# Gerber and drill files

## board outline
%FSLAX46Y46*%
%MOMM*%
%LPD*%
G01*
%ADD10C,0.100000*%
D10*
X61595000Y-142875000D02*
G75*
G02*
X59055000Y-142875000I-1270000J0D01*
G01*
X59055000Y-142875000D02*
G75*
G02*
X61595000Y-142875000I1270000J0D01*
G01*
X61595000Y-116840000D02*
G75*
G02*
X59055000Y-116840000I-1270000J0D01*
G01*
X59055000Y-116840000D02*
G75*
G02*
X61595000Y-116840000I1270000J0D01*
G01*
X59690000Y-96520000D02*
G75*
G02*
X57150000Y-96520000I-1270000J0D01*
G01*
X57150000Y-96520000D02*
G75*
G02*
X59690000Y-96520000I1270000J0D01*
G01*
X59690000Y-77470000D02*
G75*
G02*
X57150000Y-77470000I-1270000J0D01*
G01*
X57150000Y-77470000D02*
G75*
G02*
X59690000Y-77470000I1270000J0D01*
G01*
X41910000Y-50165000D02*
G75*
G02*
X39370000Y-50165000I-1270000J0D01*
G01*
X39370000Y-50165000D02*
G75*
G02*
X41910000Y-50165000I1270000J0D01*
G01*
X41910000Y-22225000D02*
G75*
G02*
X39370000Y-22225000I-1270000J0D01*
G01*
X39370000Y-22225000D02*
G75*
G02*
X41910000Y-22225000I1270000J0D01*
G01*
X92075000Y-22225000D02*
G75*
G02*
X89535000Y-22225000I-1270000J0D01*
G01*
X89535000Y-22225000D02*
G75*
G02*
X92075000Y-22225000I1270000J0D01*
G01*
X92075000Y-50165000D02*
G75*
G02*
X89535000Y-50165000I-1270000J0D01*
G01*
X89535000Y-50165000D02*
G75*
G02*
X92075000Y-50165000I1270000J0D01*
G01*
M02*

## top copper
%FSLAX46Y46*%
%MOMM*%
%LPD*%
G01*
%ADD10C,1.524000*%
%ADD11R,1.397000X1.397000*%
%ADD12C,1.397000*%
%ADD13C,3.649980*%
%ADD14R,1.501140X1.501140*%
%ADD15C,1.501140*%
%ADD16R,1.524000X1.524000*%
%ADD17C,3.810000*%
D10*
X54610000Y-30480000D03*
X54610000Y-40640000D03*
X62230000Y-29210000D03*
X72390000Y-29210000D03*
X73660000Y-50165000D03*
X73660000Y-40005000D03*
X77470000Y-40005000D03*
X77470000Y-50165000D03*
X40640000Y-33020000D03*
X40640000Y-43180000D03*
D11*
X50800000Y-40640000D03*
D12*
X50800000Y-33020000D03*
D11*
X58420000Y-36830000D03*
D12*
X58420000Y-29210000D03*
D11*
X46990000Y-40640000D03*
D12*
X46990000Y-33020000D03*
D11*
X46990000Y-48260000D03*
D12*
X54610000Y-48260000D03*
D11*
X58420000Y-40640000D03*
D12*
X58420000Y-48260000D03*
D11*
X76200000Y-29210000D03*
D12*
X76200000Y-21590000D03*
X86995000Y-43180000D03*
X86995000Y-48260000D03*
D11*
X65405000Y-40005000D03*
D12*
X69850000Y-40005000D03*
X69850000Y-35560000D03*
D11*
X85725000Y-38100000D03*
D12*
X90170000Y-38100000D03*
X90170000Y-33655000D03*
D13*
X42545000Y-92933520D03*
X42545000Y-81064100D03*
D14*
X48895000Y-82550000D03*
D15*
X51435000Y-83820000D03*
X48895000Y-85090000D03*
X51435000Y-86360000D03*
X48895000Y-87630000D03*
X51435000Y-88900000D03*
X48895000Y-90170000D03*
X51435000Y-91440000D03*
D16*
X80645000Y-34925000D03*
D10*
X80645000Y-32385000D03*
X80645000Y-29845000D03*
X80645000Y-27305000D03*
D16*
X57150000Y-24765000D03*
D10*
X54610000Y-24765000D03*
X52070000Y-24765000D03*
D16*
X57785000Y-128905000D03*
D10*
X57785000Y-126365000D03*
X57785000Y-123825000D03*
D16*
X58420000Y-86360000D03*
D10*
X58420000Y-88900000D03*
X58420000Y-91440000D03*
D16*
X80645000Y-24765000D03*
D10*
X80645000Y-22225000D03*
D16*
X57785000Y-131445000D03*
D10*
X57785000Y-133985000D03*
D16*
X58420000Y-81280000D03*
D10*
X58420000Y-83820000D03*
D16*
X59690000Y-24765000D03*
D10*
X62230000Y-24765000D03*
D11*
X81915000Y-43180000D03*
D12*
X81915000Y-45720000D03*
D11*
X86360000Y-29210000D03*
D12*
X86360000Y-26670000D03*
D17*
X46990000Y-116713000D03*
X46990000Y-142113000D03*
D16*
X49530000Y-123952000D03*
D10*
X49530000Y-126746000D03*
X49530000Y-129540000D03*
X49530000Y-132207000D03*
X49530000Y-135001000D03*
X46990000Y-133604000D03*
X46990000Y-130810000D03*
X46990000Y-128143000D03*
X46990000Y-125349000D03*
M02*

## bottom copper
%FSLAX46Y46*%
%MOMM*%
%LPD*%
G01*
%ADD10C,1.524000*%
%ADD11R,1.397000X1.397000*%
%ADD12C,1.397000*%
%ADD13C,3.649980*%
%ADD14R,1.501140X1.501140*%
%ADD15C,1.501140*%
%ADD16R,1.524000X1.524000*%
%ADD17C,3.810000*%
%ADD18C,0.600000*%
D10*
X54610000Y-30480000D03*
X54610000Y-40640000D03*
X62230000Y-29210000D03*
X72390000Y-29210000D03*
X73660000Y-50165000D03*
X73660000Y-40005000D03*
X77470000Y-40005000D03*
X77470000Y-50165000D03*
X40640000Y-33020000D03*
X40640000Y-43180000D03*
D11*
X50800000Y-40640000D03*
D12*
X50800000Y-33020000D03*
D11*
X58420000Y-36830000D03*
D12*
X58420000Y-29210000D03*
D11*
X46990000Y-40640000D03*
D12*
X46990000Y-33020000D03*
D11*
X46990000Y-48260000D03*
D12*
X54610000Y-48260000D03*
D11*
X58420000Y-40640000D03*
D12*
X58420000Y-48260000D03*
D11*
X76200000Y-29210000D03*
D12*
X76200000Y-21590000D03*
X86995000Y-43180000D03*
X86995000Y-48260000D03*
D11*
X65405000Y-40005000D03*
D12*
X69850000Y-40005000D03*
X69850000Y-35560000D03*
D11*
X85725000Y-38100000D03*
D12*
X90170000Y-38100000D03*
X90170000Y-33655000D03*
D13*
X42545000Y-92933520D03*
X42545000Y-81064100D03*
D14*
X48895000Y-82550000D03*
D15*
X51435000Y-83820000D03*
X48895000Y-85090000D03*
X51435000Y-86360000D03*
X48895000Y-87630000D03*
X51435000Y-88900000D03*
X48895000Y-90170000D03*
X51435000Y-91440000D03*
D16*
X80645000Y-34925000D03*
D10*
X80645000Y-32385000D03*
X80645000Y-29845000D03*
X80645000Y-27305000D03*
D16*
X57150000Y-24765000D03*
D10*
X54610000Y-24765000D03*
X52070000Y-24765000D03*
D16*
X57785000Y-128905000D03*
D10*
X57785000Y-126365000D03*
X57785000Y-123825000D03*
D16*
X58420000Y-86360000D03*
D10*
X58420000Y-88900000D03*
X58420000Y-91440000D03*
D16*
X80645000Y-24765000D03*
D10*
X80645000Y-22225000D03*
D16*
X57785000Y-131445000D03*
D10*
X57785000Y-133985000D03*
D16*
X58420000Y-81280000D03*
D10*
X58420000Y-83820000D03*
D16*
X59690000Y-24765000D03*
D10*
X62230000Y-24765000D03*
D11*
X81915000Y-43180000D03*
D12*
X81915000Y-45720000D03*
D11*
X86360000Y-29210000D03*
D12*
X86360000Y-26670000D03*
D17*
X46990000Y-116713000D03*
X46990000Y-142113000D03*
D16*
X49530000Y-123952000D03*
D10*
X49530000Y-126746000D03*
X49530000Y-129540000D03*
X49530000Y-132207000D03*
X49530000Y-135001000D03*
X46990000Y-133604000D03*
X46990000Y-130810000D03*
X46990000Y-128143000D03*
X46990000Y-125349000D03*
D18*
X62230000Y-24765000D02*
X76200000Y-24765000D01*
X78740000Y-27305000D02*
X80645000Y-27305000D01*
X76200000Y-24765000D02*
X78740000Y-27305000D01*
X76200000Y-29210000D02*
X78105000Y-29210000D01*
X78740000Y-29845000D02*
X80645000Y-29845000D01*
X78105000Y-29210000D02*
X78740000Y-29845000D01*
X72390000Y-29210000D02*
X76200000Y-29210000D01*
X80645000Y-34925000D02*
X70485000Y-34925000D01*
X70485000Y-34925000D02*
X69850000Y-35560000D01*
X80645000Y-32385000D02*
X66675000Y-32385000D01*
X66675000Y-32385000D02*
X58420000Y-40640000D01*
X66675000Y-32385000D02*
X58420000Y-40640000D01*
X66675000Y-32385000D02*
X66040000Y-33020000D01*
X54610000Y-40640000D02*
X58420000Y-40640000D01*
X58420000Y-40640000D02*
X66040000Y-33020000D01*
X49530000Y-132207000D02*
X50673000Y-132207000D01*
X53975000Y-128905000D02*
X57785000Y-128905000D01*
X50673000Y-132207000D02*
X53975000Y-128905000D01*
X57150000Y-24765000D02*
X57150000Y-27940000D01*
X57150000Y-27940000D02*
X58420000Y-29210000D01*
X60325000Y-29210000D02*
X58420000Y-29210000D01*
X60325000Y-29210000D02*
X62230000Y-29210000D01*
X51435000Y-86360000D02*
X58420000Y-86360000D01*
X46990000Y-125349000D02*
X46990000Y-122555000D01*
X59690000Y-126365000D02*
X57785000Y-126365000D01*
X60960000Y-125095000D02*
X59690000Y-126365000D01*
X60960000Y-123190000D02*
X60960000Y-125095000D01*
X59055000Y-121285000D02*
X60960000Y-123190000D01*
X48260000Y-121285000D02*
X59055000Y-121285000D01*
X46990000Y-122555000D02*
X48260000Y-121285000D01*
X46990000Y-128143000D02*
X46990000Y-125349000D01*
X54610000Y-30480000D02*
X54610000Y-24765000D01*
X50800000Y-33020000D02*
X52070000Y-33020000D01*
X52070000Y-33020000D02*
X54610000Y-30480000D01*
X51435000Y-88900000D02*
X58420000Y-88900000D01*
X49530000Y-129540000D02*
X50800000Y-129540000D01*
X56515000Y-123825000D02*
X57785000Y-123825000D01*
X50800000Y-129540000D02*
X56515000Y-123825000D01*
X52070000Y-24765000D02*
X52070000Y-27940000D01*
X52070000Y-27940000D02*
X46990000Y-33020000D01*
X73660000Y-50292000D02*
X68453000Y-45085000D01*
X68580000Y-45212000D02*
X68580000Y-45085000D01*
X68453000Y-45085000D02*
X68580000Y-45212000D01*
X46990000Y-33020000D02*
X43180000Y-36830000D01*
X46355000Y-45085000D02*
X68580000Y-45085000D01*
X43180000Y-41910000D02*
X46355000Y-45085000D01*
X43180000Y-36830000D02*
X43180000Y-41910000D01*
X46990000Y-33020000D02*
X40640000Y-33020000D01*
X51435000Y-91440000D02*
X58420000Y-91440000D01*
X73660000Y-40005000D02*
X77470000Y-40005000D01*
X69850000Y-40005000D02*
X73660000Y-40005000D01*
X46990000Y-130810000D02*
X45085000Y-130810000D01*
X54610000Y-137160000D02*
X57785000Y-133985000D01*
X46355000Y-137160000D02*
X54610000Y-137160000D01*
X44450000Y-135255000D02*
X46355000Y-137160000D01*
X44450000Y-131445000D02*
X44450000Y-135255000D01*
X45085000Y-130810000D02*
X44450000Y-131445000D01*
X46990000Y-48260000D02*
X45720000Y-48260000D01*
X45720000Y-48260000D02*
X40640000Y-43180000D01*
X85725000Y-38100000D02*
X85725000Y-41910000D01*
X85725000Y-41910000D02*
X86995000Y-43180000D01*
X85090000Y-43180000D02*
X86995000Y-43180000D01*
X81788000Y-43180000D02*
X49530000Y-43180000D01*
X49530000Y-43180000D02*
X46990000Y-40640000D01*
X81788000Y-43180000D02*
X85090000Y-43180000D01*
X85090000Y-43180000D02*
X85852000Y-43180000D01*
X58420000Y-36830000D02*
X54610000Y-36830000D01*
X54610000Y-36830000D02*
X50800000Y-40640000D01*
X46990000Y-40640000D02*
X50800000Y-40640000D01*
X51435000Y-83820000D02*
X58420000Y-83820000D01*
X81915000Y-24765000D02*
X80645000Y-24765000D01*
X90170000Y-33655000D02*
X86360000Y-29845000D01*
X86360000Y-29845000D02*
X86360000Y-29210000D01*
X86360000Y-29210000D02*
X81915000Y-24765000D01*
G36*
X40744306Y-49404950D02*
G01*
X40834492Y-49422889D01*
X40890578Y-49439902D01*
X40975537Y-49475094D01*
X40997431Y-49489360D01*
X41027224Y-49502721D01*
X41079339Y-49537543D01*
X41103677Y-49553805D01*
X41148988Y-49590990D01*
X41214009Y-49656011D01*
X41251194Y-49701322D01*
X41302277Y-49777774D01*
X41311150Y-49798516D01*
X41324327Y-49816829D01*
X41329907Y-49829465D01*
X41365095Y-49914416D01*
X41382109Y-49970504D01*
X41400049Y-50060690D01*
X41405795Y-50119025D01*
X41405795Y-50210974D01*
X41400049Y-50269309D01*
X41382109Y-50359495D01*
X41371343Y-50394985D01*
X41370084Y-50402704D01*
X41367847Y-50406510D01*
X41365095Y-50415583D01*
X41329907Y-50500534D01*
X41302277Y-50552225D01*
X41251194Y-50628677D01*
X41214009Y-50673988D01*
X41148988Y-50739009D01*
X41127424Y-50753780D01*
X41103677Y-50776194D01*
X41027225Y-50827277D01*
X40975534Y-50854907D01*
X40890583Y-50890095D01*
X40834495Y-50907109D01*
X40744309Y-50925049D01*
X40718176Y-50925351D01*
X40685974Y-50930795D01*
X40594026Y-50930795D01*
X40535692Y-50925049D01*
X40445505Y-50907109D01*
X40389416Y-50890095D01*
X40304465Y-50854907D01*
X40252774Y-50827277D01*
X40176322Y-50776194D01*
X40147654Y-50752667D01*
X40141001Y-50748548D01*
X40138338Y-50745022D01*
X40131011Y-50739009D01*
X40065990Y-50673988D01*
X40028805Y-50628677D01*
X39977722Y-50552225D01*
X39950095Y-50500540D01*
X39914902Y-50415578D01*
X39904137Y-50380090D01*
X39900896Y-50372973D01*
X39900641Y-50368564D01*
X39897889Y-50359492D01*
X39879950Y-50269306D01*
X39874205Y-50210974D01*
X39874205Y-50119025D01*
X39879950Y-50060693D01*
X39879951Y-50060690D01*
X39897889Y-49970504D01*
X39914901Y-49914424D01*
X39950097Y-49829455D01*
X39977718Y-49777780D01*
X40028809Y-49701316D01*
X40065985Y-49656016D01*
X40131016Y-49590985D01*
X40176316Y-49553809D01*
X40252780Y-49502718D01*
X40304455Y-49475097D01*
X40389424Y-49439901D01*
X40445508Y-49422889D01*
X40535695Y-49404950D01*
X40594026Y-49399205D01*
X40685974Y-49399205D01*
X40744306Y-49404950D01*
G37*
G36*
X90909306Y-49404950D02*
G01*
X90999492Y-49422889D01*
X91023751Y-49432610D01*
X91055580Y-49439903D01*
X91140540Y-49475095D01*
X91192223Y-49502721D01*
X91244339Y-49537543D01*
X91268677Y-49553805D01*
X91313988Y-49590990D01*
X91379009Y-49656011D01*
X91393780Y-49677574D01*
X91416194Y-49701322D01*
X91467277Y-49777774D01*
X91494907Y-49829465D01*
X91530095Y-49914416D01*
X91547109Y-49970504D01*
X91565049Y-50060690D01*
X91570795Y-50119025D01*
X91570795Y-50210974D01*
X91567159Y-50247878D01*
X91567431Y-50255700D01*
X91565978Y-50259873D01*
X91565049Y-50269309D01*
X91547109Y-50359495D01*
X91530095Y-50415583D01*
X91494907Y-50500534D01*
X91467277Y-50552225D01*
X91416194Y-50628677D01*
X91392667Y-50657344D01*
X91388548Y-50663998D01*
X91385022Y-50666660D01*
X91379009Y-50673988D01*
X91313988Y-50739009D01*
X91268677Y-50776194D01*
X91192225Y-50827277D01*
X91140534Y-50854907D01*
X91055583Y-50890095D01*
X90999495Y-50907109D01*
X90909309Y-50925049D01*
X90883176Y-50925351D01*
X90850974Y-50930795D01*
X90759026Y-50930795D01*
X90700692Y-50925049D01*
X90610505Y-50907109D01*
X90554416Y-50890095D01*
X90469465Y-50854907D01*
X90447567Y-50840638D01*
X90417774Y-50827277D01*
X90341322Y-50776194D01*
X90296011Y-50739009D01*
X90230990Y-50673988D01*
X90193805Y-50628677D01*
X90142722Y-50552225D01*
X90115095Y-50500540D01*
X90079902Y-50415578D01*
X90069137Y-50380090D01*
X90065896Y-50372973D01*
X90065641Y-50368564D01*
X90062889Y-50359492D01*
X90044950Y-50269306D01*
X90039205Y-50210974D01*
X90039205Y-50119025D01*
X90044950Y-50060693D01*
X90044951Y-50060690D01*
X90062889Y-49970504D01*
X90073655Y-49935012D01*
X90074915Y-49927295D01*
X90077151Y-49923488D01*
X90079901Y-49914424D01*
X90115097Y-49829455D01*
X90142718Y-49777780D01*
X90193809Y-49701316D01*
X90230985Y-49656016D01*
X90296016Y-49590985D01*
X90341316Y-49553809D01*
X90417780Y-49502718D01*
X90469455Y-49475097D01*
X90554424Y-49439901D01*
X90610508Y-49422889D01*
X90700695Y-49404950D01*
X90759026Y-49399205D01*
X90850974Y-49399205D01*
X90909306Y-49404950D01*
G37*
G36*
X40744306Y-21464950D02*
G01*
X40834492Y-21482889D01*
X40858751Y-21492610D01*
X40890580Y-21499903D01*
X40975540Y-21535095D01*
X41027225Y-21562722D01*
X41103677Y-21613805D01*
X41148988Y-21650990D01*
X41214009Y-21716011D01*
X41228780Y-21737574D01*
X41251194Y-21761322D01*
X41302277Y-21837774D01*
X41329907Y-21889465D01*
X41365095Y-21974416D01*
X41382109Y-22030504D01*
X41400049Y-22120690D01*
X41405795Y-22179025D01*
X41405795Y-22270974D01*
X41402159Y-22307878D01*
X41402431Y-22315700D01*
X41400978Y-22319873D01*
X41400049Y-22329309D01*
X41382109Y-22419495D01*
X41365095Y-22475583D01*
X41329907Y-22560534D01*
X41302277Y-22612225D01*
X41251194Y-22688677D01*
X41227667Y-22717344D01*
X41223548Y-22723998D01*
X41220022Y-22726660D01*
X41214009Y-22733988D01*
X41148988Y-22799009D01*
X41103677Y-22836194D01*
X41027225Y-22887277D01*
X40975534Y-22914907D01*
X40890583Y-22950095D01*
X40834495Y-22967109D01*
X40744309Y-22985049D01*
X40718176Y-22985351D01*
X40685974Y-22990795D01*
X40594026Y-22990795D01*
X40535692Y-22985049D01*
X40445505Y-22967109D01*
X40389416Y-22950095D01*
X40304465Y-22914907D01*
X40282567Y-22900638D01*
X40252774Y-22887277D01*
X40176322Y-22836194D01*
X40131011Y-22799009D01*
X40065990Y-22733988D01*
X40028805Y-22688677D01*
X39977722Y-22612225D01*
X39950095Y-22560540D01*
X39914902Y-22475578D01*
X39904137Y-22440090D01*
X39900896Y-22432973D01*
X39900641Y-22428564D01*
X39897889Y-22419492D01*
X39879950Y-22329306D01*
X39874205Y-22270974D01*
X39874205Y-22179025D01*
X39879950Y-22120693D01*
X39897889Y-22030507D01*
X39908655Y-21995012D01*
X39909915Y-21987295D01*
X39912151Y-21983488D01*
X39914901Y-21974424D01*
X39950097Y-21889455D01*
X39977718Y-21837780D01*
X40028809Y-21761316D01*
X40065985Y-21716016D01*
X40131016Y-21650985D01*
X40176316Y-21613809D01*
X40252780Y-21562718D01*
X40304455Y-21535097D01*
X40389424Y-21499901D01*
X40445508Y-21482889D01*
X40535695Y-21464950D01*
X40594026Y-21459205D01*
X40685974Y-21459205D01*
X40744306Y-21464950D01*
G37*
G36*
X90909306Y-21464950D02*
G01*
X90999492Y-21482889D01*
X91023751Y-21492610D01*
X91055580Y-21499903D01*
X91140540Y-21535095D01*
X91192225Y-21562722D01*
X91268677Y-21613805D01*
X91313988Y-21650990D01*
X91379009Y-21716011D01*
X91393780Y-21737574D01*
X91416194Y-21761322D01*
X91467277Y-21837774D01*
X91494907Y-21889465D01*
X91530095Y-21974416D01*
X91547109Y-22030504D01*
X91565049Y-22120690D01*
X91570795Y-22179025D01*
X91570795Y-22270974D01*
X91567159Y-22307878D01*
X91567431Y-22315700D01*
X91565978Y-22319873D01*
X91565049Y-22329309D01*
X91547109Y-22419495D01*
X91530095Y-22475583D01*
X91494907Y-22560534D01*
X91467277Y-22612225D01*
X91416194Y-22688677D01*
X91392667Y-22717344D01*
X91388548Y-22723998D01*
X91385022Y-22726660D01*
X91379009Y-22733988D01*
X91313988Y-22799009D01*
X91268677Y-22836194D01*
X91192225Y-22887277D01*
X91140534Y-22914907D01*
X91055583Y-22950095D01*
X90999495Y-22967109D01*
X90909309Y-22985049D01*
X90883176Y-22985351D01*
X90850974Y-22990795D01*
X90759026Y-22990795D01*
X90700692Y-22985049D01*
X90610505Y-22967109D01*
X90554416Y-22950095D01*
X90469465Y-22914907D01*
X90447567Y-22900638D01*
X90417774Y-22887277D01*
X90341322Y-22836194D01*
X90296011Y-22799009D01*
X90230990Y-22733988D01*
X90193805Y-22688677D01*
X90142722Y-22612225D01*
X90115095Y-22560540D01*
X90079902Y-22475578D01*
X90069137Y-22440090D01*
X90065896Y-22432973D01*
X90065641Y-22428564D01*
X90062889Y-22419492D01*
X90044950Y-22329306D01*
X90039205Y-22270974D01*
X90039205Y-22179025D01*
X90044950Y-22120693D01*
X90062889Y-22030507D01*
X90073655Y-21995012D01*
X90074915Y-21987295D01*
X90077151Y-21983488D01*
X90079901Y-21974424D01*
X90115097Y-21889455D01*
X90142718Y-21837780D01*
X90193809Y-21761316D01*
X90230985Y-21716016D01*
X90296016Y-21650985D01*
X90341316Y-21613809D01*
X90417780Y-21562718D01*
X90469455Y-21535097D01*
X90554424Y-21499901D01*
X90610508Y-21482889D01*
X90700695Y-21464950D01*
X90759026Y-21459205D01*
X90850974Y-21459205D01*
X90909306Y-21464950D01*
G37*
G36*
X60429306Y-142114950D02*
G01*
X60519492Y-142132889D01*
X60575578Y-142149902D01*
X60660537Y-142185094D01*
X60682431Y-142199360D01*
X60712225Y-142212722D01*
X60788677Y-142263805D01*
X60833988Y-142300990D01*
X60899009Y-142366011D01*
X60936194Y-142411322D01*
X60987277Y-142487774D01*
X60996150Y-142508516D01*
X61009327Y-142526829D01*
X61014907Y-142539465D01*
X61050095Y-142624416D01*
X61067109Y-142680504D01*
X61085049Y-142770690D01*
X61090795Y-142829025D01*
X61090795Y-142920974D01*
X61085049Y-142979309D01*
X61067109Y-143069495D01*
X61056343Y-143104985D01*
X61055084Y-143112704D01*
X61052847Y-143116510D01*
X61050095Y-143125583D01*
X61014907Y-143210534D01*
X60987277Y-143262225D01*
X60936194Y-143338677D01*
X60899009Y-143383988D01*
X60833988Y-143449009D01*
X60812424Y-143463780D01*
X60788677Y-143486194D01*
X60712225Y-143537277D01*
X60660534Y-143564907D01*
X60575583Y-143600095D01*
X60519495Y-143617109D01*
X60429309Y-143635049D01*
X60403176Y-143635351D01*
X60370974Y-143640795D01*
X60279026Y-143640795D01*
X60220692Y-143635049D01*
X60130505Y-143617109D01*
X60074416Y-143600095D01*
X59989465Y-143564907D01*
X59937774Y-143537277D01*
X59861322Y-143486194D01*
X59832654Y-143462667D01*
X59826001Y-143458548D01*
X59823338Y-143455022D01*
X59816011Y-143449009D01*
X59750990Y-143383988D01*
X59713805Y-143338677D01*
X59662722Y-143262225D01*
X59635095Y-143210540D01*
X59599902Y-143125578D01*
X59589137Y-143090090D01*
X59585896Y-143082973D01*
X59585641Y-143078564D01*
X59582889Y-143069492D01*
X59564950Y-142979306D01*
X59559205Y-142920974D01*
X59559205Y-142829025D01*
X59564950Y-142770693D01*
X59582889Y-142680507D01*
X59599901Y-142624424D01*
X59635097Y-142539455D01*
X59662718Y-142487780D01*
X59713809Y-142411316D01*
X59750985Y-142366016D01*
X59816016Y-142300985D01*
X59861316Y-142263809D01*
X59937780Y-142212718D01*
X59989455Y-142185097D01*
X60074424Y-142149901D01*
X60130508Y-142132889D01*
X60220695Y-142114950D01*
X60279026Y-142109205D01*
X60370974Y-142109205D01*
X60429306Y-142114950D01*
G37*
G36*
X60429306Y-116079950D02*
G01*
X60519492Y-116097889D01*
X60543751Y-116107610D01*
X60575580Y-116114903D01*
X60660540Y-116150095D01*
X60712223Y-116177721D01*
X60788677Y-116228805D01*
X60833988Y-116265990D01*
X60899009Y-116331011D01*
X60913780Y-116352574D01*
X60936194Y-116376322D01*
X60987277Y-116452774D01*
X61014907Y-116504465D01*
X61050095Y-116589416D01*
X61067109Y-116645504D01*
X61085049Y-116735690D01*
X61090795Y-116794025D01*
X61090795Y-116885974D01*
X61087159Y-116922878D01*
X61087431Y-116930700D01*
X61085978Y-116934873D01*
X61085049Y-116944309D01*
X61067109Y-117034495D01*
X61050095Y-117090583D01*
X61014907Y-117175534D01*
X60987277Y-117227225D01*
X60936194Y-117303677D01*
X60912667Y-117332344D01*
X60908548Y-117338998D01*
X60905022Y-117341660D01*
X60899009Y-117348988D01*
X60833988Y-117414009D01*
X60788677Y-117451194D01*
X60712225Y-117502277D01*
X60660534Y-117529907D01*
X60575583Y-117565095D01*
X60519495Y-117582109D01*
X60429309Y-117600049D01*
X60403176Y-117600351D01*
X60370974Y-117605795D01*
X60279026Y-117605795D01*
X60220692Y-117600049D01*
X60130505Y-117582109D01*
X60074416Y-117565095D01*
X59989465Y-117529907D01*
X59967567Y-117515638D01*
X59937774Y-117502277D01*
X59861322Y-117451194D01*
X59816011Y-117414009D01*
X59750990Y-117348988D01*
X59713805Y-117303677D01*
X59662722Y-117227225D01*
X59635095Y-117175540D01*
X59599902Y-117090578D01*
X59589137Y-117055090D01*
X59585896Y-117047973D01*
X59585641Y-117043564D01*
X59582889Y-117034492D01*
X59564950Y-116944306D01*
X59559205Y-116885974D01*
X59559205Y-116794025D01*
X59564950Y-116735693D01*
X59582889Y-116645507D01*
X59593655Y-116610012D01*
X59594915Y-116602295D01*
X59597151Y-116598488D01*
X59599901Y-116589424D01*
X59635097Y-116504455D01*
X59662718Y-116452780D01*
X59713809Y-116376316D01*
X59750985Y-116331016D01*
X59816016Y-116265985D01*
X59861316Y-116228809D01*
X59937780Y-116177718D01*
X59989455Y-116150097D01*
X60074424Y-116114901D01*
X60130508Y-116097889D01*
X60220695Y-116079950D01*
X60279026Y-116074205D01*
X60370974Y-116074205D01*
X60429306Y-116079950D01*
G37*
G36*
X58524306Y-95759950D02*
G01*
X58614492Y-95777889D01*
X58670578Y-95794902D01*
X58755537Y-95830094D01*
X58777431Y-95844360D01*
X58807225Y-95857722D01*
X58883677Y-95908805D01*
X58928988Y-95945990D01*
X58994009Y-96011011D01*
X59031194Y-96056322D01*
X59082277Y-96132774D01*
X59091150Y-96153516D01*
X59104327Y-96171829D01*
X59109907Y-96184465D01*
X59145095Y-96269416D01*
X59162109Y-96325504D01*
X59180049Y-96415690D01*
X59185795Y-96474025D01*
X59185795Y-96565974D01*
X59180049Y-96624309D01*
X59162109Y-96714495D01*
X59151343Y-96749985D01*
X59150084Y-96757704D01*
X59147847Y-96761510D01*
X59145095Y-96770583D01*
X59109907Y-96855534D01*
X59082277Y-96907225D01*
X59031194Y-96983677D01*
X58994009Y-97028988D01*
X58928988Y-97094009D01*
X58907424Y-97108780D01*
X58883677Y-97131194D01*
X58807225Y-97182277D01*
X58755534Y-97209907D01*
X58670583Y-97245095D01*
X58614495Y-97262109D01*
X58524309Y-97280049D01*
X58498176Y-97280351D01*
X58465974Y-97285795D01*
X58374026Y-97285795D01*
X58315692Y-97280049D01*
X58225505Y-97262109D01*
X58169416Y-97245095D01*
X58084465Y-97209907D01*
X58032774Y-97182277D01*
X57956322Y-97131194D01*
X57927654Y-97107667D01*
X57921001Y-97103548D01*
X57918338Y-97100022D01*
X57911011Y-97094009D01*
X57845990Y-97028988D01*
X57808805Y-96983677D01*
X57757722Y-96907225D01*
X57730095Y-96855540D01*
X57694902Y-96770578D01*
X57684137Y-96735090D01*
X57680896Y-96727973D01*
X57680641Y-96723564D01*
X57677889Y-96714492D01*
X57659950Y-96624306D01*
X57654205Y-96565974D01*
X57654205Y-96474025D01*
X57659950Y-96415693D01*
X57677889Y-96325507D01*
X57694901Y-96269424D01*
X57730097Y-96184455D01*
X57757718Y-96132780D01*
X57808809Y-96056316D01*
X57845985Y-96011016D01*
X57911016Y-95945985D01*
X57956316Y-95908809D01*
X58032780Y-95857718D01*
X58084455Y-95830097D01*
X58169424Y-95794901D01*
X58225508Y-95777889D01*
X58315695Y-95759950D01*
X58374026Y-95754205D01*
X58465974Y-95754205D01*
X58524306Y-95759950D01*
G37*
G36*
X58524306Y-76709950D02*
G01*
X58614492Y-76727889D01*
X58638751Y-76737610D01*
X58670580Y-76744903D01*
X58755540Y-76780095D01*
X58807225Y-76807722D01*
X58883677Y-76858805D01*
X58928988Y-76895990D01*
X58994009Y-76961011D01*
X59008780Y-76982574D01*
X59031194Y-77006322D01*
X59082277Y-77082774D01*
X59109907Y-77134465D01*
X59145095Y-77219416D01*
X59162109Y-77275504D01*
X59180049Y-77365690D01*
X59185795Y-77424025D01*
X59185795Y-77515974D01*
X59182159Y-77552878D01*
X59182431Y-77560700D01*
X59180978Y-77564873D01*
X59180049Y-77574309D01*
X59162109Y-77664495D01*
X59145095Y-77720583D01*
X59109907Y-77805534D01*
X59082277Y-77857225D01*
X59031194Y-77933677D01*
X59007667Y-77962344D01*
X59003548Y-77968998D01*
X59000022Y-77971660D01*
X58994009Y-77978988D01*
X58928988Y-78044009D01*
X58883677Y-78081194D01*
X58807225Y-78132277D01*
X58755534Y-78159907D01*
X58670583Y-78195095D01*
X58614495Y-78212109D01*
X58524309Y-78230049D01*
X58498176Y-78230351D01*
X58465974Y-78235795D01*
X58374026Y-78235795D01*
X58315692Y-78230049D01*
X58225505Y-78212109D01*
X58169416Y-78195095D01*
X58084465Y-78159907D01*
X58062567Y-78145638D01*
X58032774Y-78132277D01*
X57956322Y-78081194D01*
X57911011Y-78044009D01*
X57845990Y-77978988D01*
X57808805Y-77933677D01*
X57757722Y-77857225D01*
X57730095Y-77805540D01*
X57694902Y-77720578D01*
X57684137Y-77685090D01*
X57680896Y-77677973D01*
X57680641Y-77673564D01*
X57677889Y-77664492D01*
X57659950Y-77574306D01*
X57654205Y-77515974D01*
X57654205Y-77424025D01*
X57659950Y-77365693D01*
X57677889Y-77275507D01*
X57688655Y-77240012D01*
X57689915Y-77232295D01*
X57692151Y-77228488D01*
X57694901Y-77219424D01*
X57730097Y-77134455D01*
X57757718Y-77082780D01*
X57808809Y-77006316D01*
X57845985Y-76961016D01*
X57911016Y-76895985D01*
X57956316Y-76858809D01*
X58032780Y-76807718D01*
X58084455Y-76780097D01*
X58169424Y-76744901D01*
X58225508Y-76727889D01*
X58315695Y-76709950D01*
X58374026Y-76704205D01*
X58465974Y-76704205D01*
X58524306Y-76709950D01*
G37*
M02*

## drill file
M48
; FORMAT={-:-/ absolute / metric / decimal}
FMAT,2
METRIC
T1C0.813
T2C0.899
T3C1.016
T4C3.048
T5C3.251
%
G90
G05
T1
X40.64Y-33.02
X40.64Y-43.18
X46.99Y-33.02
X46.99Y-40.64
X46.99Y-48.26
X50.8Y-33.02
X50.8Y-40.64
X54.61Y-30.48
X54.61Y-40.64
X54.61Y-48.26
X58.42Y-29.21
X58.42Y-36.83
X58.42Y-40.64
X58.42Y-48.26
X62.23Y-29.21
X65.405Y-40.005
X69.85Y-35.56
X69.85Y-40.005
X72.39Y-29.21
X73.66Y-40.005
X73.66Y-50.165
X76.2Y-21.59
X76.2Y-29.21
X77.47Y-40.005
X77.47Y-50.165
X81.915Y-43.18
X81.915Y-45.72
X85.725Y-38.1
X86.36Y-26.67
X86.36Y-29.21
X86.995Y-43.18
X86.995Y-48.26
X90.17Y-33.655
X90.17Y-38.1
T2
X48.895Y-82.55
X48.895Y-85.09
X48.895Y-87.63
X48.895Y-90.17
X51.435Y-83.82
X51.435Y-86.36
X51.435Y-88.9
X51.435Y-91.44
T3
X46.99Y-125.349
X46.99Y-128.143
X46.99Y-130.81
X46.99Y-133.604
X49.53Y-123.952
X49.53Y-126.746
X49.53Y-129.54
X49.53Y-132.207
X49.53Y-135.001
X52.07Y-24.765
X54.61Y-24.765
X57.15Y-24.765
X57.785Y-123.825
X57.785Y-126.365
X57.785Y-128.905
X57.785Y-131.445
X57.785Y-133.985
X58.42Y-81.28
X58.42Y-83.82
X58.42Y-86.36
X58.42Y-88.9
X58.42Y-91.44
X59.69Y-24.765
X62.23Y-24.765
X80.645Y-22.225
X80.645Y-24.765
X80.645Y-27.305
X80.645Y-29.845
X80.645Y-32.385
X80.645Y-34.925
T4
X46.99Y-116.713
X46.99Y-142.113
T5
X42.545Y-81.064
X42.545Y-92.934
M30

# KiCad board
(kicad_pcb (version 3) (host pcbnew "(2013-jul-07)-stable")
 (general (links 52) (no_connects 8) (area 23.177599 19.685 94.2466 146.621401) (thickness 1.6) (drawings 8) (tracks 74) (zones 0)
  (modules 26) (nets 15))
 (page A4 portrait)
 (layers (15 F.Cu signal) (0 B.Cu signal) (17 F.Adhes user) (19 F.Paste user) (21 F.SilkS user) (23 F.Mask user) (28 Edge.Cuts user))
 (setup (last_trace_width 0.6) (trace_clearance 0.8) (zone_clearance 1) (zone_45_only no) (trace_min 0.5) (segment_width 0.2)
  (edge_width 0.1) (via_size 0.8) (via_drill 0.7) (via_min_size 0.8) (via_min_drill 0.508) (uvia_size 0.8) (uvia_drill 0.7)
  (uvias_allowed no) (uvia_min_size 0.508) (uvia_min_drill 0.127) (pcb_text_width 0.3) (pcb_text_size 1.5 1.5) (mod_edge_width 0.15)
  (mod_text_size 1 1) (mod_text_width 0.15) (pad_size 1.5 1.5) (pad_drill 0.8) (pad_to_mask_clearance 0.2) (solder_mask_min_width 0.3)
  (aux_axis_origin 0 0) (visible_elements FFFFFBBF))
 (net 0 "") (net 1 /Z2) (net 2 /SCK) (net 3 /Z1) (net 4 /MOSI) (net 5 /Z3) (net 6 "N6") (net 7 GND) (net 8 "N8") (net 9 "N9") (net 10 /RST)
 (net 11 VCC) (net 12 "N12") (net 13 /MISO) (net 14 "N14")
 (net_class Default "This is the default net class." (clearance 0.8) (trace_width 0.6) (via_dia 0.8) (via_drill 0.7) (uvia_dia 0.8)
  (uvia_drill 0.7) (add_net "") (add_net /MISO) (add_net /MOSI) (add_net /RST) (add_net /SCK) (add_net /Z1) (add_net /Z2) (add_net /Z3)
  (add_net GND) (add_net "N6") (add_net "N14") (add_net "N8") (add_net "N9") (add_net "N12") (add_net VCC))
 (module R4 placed (layer F.Cu) (at 54.61 35.56 270) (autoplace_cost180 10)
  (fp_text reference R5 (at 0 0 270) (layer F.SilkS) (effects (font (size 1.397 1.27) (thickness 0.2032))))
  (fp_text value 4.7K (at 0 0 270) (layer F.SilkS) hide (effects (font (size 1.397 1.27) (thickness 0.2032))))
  (pad 1 thru_hole circle (at -5.08 0 270) (size 1.524 1.524) (drill 0.8128) (layers *.Cu *.Mask F.SilkS) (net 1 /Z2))
  (pad 2 thru_hole circle (at 5.08 0 270) (size 1.524 1.524) (drill 0.8128) (layers *.Cu *.Mask F.SilkS) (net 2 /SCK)))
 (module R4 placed (layer F.Cu) (at 67.31 29.21) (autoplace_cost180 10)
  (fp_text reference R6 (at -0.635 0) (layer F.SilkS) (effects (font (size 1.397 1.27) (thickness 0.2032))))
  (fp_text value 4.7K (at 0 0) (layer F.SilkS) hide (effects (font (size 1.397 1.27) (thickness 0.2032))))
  (pad 1 thru_hole circle (at -5.08 0) (size 1.524 1.524) (drill 0.8128) (layers *.Cu *.Mask F.SilkS) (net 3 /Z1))
  (pad 2 thru_hole circle (at 5.08 0) (size 1.524 1.524) (drill 0.8128) (layers *.Cu *.Mask F.SilkS) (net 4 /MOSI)))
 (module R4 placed (layer F.Cu) (at 73.66 45.085 90) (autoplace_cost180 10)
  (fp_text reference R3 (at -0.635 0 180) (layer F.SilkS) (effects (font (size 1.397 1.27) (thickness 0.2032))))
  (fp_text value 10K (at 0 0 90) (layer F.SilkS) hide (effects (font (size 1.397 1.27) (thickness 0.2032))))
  (pad 1 thru_hole circle (at -5.08 0 90) (size 1.524 1.524) (drill 0.8128) (layers *.Cu *.Mask F.SilkS) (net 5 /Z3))
  (pad 2 thru_hole circle (at 5.08 0 90) (size 1.524 1.524) (drill 0.8128) (layers *.Cu *.Mask F.SilkS) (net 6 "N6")))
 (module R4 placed (layer F.Cu) (at 77.47 45.085 270) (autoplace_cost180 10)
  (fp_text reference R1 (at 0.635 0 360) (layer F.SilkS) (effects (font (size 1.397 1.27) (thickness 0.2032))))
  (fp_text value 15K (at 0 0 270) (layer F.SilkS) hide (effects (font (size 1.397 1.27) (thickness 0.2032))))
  (pad 1 thru_hole circle (at -5.08 0 270) (size 1.524 1.524) (drill 0.8128) (layers *.Cu *.Mask F.SilkS) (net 6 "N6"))
  (pad 2 thru_hole circle (at 5.08 0 270) (size 1.524 1.524) (drill 0.8128) (layers *.Cu *.Mask F.SilkS) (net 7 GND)))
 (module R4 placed (layer F.Cu) (at 40.64 38.1 270) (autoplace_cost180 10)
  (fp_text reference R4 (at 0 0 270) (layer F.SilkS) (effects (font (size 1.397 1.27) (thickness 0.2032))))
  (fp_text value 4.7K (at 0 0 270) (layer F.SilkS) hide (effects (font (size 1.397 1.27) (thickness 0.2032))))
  (pad 1 thru_hole circle (at -5.08 0 270) (size 1.524 1.524) (drill 0.8128) (layers *.Cu *.Mask F.SilkS) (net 5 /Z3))
  (pad 2 thru_hole circle (at 5.08 0 270) (size 1.524 1.524) (drill 0.8128) (layers *.Cu *.Mask F.SilkS) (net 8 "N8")))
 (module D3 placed (layer F.Cu) (at 50.8 36.83 270)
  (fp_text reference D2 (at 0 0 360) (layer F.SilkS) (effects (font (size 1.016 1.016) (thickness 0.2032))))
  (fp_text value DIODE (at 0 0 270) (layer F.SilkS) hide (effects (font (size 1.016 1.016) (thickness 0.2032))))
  (pad 2 thru_hole rect (at 3.81 0 270) (size 1.397 1.397) (drill 0.8128) (layers *.Cu *.Mask F.SilkS) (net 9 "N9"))
  (pad 1 thru_hole circle (at -3.81 0 270) (size 1.397 1.397) (drill 0.8128) (layers *.Cu *.Mask F.SilkS) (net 1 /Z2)))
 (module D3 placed (layer F.Cu) (at 58.42 33.02 270)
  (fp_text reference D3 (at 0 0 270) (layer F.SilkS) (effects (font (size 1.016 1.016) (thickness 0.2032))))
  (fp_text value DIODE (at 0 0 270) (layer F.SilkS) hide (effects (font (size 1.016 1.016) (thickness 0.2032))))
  (pad 2 thru_hole rect (at 3.81 0 270) (size 1.397 1.397) (drill 0.8128) (layers *.Cu *.Mask F.SilkS) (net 9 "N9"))
  (pad 1 thru_hole circle (at -3.81 0 270) (size 1.397 1.397) (drill 0.8128) (layers *.Cu *.Mask F.SilkS) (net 3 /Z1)))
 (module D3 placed (layer F.Cu) (at 46.99 36.83 270)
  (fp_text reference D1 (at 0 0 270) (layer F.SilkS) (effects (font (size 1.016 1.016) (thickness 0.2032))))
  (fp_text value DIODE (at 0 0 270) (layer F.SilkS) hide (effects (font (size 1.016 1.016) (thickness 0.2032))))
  (pad 2 thru_hole rect (at 3.81 0 270) (size 1.397 1.397) (drill 0.8128) (layers *.Cu *.Mask F.SilkS) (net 9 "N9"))
  (pad 1 thru_hole circle (at -3.81 0 270) (size 1.397 1.397) (drill 0.8128) (layers *.Cu *.Mask F.SilkS) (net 5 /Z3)))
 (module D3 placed (layer F.Cu) (at 50.8 48.26 180)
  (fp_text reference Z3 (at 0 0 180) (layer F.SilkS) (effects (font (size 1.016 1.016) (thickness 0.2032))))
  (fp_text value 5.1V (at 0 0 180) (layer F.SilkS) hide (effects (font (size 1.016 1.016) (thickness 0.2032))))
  (pad 2 thru_hole rect (at 3.81 0 180) (size 1.397 1.397) (drill 0.8128) (layers *.Cu *.Mask F.SilkS) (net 8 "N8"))
  (pad 1 thru_hole circle (at -3.81 0 180) (size 1.397 1.397) (drill 0.8128) (layers *.Cu *.Mask F.SilkS) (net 7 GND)))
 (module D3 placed (layer F.Cu) (at 58.42 44.45 90)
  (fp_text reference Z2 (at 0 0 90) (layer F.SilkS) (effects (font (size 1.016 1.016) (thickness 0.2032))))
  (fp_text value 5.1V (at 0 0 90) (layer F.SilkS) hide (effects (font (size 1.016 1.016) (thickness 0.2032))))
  (pad 2 thru_hole rect (at 3.81 0 90) (size 1.397 1.397) (drill 0.8128) (layers *.Cu *.Mask F.SilkS) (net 2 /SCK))
  (pad 1 thru_hole circle (at -3.81 0 90) (size 1.397 1.397) (drill 0.8128) (layers *.Cu *.Mask F.SilkS) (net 7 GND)))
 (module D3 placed (layer F.Cu) (at 76.2 25.4 270)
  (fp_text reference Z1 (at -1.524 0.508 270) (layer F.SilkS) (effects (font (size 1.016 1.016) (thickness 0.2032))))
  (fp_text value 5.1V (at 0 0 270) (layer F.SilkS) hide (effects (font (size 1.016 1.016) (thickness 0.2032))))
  (pad 2 thru_hole rect (at 3.81 0 270) (size 1.397 1.397) (drill 0.8128) (layers *.Cu *.Mask F.SilkS) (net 4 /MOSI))
  (pad 1 thru_hole circle (at -3.81 0 270) (size 1.397 1.397) (drill 0.8128) (layers *.Cu *.Mask F.SilkS) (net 7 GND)))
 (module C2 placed (layer F.Cu) (at 86.995 45.72 270)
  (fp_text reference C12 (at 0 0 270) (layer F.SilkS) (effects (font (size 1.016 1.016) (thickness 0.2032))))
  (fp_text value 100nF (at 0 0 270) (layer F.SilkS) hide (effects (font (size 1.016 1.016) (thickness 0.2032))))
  (pad 1 thru_hole circle (at -2.54 0 270) (size 1.397 1.397) (drill 0.8128) (layers *.Cu *.Mask F.SilkS) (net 9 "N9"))
  (pad 2 thru_hole circle (at 2.54 0 270) (size 1.397 1.397) (drill 0.8128) (layers *.Cu *.Mask F.SilkS) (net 7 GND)))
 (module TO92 (layer F.Cu) (at 67.31 37.465 180)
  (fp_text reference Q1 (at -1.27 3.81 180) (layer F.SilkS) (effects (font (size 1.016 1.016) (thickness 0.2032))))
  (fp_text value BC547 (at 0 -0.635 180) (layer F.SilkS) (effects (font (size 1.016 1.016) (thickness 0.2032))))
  (pad 1 thru_hole rect (at 1.905 -2.54 180) (size 1.397 1.397) (drill 0.8128) (layers *.Cu *.Mask F.SilkS) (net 7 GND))
  (pad 2 thru_hole circle (at -2.54 -2.54 180) (size 1.397 1.397) (drill 0.8128) (layers *.Cu *.Mask F.SilkS) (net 6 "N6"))
  (pad 3 thru_hole circle (at -2.54 1.905 180) (size 1.397 1.397) (drill 0.8128) (layers *.Cu *.Mask F.SilkS) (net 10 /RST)))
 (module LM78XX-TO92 (layer F.Cu) (at 87.63 35.56 180)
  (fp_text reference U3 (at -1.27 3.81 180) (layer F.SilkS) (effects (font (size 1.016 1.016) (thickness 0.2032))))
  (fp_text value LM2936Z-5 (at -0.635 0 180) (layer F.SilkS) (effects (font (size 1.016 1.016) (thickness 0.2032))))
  (pad VI thru_hole rect (at 1.905 -2.54 180) (size 1.397 1.397) (drill 0.8128) (layers *.Cu *.Mask F.SilkS) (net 9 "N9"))
  (pad GND thru_hole circle (at -2.54 -2.54 180) (size 1.397 1.397) (drill 0.8128) (layers *.Cu *.Mask F.SilkS) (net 7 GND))
  (pad VO thru_hole circle (at -2.54 1.905 180) (size 1.397 1.397) (drill 0.8128) (layers *.Cu *.Mask F.SilkS) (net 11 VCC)))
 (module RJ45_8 (layer F.Cu) (at 42.545 86.995 270)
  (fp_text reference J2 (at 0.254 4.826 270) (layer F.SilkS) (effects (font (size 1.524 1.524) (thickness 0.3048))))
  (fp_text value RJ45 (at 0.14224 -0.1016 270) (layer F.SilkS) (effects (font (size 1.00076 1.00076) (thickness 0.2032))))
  (pad Hole np_thru_hole circle (at 5.93852 0 270) (size 3.64998 3.64998) (drill 3.2512) (layers *.Cu *.SilkS *.Mask))
  (pad Hole np_thru_hole circle (at -5.9309 0 270) (size 3.64998 3.64998) (drill 3.2512) (layers *.Cu *.SilkS *.Mask))
  (pad 1 thru_hole rect (at -4.445 -6.35 270) (size 1.50114 1.50114) (drill 0.89916) (layers *.Cu *.Mask F.SilkS) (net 7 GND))
  (pad 2 thru_hole circle (at -3.175 -8.89 270) (size 1.50114 1.50114) (drill 0.89916) (layers *.Cu *.Mask F.SilkS) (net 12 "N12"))
  (pad 3 thru_hole circle (at -1.905 -6.35 270) (size 1.50114 1.50114) (drill 0.89916) (layers *.Cu *.Mask F.SilkS))
  (pad 4 thru_hole circle (at -0.635 -8.89 270) (size 1.50114 1.50114) (drill 0.89916) (layers *.Cu *.Mask F.SilkS) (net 3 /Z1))
  (pad 5 thru_hole circle (at 0.635 -6.35 270) (size 1.50114 1.50114) (drill 0.89916) (layers *.Cu *.Mask F.SilkS))
  (pad 6 thru_hole circle (at 1.905 -8.89 270) (size 1.50114 1.50114) (drill 0.89916) (layers *.Cu *.Mask F.SilkS) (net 1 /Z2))
  (pad 7 thru_hole circle (at 3.175 -6.35 270) (size 1.50114 1.50114) (drill 0.89916) (layers *.Cu *.Mask F.SilkS))
  (pad 8 thru_hole circle (at 4.445 -8.89 270) (size 1.50114 1.50114) (drill 0.89916) (layers *.Cu *.Mask F.SilkS) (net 5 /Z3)))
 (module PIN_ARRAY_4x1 (layer F.Cu) (at 80.645 31.115 90)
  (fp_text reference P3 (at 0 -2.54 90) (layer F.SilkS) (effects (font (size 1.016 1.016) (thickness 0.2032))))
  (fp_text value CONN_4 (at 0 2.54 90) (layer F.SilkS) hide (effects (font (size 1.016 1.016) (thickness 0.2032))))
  (pad 1 thru_hole rect (at -3.81 0 90) (size 1.524 1.524) (drill 1.016) (layers *.Cu *.Mask F.SilkS) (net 10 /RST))
  (pad 2 thru_hole circle (at -1.27 0 90) (size 1.524 1.524) (drill 1.016) (layers *.Cu *.Mask F.SilkS) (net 2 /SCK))
  (pad 3 thru_hole circle (at 1.27 0 90) (size 1.524 1.524) (drill 1.016) (layers *.Cu *.Mask F.SilkS) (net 4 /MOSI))
  (pad 4 thru_hole circle (at 3.81 0 90) (size 1.524 1.524) (drill 1.016) (layers *.Cu *.Mask F.SilkS) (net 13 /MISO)))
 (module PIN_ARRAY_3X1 (layer F.Cu) (at 54.61 24.765 180)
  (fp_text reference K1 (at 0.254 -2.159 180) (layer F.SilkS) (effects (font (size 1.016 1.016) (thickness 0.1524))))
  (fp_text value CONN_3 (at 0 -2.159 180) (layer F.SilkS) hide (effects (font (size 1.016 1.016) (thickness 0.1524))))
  (pad 1 thru_hole rect (at -2.54 0 180) (size 1.524 1.524) (drill 1.016) (layers *.Cu *.Mask F.SilkS) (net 3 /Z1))
  (pad 2 thru_hole circle (at 0 0 180) (size 1.524 1.524) (drill 1.016) (layers *.Cu *.Mask F.SilkS) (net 1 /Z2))
  (pad 3 thru_hole circle (at 2.54 0 180) (size 1.524 1.524) (drill 1.016) (layers *.Cu *.Mask F.SilkS) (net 5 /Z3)))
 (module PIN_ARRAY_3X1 (layer F.Cu) (at 57.785 126.365 90)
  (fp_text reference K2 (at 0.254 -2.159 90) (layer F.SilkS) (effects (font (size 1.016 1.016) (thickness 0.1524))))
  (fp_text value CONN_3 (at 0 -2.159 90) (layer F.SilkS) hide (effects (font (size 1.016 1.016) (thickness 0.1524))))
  (pad 1 thru_hole rect (at -2.54 0 90) (size 1.524 1.524) (drill 1.016) (layers *.Cu *.Mask F.SilkS) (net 3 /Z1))
  (pad 2 thru_hole circle (at 0 0 90) (size 1.524 1.524) (drill 1.016) (layers *.Cu *.Mask F.SilkS) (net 1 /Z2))
  (pad 3 thru_hole circle (at 2.54 0 90) (size 1.524 1.524) (drill 1.016) (layers *.Cu *.Mask F.SilkS) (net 5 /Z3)))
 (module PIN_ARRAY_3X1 (layer F.Cu) (at 58.42 88.9 270)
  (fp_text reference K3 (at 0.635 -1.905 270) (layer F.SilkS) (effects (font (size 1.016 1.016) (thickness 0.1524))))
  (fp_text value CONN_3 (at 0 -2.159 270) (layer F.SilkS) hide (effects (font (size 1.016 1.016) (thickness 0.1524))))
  (pad 1 thru_hole rect (at -2.54 0 270) (size 1.524 1.524) (drill 1.016) (layers *.Cu *.Mask F.SilkS) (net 3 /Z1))
  (pad 2 thru_hole circle (at 0 0 270) (size 1.524 1.524) (drill 1.016) (layers *.Cu *.Mask F.SilkS) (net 1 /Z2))
  (pad 3 thru_hole circle (at 2.54 0 270) (size 1.524 1.524) (drill 1.016) (layers *.Cu *.Mask F.SilkS) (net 5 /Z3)))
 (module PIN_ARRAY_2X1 (layer F.Cu) (at 80.645 23.495 90)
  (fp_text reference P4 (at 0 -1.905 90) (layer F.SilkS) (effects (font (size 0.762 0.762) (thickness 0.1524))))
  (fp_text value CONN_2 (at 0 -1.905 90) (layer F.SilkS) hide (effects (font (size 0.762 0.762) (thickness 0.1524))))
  (pad 1 thru_hole rect (at -1.27 0 90) (size 1.524 1.524) (drill 1.016) (layers *.Cu *.Mask F.SilkS) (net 11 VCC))
  (pad 2 thru_hole circle (at 1.27 0 90) (size 1.524 1.524) (drill 1.016) (layers *.Cu *.Mask F.SilkS) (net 7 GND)))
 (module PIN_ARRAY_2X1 (layer F.Cu) (at 57.785 132.715 270)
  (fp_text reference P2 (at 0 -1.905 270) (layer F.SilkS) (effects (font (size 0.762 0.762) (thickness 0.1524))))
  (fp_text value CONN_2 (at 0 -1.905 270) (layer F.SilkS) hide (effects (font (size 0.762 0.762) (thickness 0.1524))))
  (pad 1 thru_hole rect (at -1.27 0 270) (size 1.524 1.524) (drill 1.016) (layers *.Cu *.Mask F.SilkS) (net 7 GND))
  (pad 2 thru_hole circle (at 1.27 0 270) (size 1.524 1.524) (drill 1.016) (layers *.Cu *.Mask F.SilkS) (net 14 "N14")))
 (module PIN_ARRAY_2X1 (layer F.Cu) (at 58.42 82.55 270)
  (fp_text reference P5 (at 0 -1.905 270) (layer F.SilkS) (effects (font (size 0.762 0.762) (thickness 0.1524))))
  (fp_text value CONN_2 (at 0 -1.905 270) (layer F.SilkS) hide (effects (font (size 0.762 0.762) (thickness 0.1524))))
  (pad 1 thru_hole rect (at -1.27 0 270) (size 1.524 1.524) (drill 1.016) (layers *.Cu *.Mask F.SilkS) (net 7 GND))
  (pad 2 thru_hole circle (at 1.27 0 270) (size 1.524 1.524) (drill 1.016) (layers *.Cu *.Mask F.SilkS) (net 12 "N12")))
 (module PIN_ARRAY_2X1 (layer F.Cu) (at 60.96 24.765)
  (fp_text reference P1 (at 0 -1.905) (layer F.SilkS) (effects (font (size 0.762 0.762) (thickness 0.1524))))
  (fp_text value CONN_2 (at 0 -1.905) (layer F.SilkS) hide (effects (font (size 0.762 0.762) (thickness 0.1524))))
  (pad 1 thru_hole rect (at -1.27 0) (size 1.524 1.524) (drill 1.016) (layers *.Cu *.Mask F.SilkS) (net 7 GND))
  (pad 2 thru_hole circle (at 1.27 0) (size 1.524 1.524) (drill 1.016) (layers *.Cu *.Mask F.SilkS) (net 13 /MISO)))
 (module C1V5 (layer F.Cu) (at 81.915 44.45 270)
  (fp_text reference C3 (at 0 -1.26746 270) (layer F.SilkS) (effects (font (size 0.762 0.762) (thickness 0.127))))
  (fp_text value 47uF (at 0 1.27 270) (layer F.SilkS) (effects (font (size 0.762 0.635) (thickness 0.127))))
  (pad 1 thru_hole rect (at -1.27 0 270) (size 1.397 1.397) (drill 0.8128) (layers *.Cu *.Mask F.SilkS) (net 9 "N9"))
  (pad 2 thru_hole circle (at 1.27 0 270) (size 1.397 1.397) (drill 0.8128) (layers *.Cu *.Mask F.SilkS) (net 7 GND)))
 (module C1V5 (layer F.Cu) (at 86.36 27.94 90)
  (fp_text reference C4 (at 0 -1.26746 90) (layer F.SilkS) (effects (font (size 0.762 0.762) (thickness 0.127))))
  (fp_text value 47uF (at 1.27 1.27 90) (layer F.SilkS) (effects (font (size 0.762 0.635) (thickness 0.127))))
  (pad 1 thru_hole rect (at -1.27 0 90) (size 1.397 1.397) (drill 0.8128) (layers *.Cu *.Mask F.SilkS) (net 11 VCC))
  (pad 2 thru_hole circle (at 1.27 0 90) (size 1.397 1.397) (drill 0.8128) (layers *.Cu *.Mask F.SilkS) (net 7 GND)))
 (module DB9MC (layer F.Cu) (at 48.26 129.54 90)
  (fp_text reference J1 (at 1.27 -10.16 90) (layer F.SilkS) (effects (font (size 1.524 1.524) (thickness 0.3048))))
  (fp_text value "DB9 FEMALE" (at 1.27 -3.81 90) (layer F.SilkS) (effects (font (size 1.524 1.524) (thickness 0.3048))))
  (pad "" thru_hole circle (at 12.827 -1.27 90) (size 3.81 3.81) (drill 3.048) (layers *.Cu *.Mask F.SilkS))
  (pad "" thru_hole circle (at -12.573 -1.27 90) (size 3.81 3.81) (drill 3.048) (layers *.Cu *.Mask F.SilkS))
  (pad 1 thru_hole rect (at 5.588 1.27 90) (size 1.524 1.524) (drill 1.016) (layers *.Cu *.Mask F.SilkS))
  (pad 2 thru_hole circle (at 2.794 1.27 90) (size 1.524 1.524) (drill 1.016) (layers *.Cu *.Mask F.SilkS))
  (pad 3 thru_hole circle (at 0 1.27 90) (size 1.524 1.524) (drill 1.016) (layers *.Cu *.Mask F.SilkS) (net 5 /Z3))
  (pad 4 thru_hole circle (at -2.667 1.27 90) (size 1.524 1.524) (drill 1.016) (layers *.Cu *.Mask F.SilkS) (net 3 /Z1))
  (pad 5 thru_hole circle (at -5.461 1.27 90) (size 1.524 1.524) (drill 1.016) (layers *.Cu *.Mask F.SilkS) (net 7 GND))
  (pad 9 thru_hole circle (at -4.064 -1.27 90) (size 1.524 1.524) (drill 1.016) (layers *.Cu *.Mask F.SilkS))
  (pad 8 thru_hole circle (at -1.27 -1.27 90) (size 1.524 1.524) (drill 1.016) (layers *.Cu *.Mask F.SilkS) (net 14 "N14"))
  (pad 7 thru_hole circle (at 1.397 -1.27 90) (size 1.524 1.524) (drill 1.016) (layers *.Cu *.Mask F.SilkS) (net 1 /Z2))
  (pad 6 thru_hole circle (at 4.191 -1.27 90) (size 1.524 1.524) (drill 1.016) (layers *.Cu *.Mask F.SilkS) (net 1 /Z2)))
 (gr_circle (center 60.325 142.875) (end 61.595 142.875) (layer Edge.Cuts) (width 0.1))
 (gr_circle (center 60.325 116.84) (end 61.595 116.84) (layer Edge.Cuts) (width 0.1))
 (gr_circle (center 58.42 96.52) (end 59.69 96.52) (layer Edge.Cuts) (width 0.1))
 (gr_circle (center 58.42 77.47) (end 59.69 77.47) (layer Edge.Cuts) (width 0.1))
 (gr_circle (center 40.64 50.165) (end 41.91 50.165) (layer Edge.Cuts) (width 0.1))
 (gr_circle (center 40.64 22.225) (end 41.91 22.225) (layer Edge.Cuts) (width 0.1))
 (gr_circle (center 90.805 22.225) (end 89.535 22.225) (layer Edge.Cuts) (width 0.1))
 (gr_circle (center 90.805 50.165) (end 89.535 50.165) (layer Edge.Cuts) (width 0.1))
 (segment (start 62.23 24.765) (end 76.2 24.765) (width 0.6) (layer B.Cu) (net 13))
 (segment (start 78.74 27.305) (end 80.645 27.305) (width 0.6) (layer B.Cu) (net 13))
 (segment (start 76.2 24.765) (end 78.74 27.305) (width 0.6) (layer B.Cu) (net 13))
 (segment (start 76.2 29.21) (end 78.105 29.21) (width 0.6) (layer B.Cu) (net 4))
 (segment (start 78.74 29.845) (end 80.645 29.845) (width 0.6) (layer B.Cu) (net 4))
 (segment (start 78.105 29.21) (end 78.74 29.845) (width 0.6) (layer B.Cu) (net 4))
 (segment (start 72.39 29.21) (end 76.2 29.21) (width 0.6) (layer B.Cu) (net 4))
 (segment (start 80.645 34.925) (end 70.485 34.925) (width 0.6) (layer B.Cu) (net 10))
 (segment (start 70.485 34.925) (end 69.85 35.56) (width 0.6) (layer B.Cu) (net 10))
 (segment (start 80.645 32.385) (end 66.675 32.385) (width 0.6) (layer B.Cu) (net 2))
 (segment (start 66.675 32.385) (end 58.42 40.64) (width 0.6) (layer B.Cu) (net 2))
 (segment (start 66.675 32.385) (end 58.42 40.64) (width 0.6) (layer B.Cu) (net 2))
 (segment (start 66.675 32.385) (end 66.04 33.02) (width 0.6) (layer B.Cu) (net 2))
 (segment (start 54.61 40.64) (end 58.42 40.64) (width 0.6) (layer B.Cu) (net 2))
 (segment (start 58.42 40.64) (end 66.04 33.02) (width 0.6) (layer B.Cu) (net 2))
 (segment (start 49.53 132.207) (end 50.673 132.207) (width 0.6) (layer B.Cu) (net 3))
 (segment (start 53.975 128.905) (end 57.785 128.905) (width 0.6) (layer B.Cu) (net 3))
 (segment (start 50.673 132.207) (end 53.975 128.905) (width 0.6) (layer B.Cu) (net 3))
 (segment (start 57.15 24.765) (end 57.15 27.94) (width 0.6) (layer B.Cu) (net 3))
 (segment (start 57.15 27.94) (end 58.42 29.21) (width 0.6) (layer B.Cu) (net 3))
 (segment (start 60.325 29.21) (end 58.42 29.21) (width 0.6) (layer B.Cu) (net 3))
 (segment (start 60.325 29.21) (end 62.23 29.21) (width 0.6) (layer B.Cu) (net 3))
 (segment (start 51.435 86.36) (end 58.42 86.36) (width 0.6) (layer B.Cu) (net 3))
 (segment (start 46.99 125.349) (end 46.99 122.555) (width 0.6) (layer B.Cu) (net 1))
 (segment (start 59.69 126.365) (end 57.785 126.365) (width 0.6) (layer B.Cu) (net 1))
 (segment (start 60.96 125.095) (end 59.69 126.365) (width 0.6) (layer B.Cu) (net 1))
 (segment (start 60.96 123.19) (end 60.96 125.095) (width 0.6) (layer B.Cu) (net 1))
 (segment (start 59.055 121.285) (end 60.96 123.19) (width 0.6) (layer B.Cu) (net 1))
 (segment (start 48.26 121.285) (end 59.055 121.285) (width 0.6) (layer B.Cu) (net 1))
 (segment (start 46.99 122.555) (end 48.26 121.285) (width 0.6) (layer B.Cu) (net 1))
 (segment (start 46.99 128.143) (end 46.99 125.349) (width 0.6) (layer B.Cu) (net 1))
 (segment (start 54.61 30.48) (end 54.61 24.765) (width 0.6) (layer B.Cu) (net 1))
 (segment (start 50.8 33.02) (end 52.07 33.02) (width 0.6) (layer B.Cu) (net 1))
 (segment (start 52.07 33.02) (end 54.61 30.48) (width 0.6) (layer B.Cu) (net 1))
 (segment (start 51.435 88.9) (end 58.42 88.9) (width 0.6) (layer B.Cu) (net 1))
 (segment (start 49.53 129.54) (end 50.8 129.54) (width 0.6) (layer B.Cu) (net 5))
 (segment (start 56.515 123.825) (end 57.785 123.825) (width 0.6) (layer B.Cu) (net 5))
 (segment (start 50.8 129.54) (end 56.515 123.825) (width 0.6) (layer B.Cu) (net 5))
 (segment (start 52.07 24.765) (end 52.07 27.94) (width 0.6) (layer B.Cu) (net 5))
 (segment (start 52.07 27.94) (end 46.99 33.02) (width 0.6) (layer B.Cu) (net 5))
 (segment (start 73.66 50.292) (end 68.453 45.085) (width 0.6) (layer B.Cu) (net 5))
 (segment (start 68.58 45.212) (end 68.58 45.085) (width 0.6) (layer B.Cu) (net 5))
 (segment (start 68.453 45.085) (end 68.58 45.212) (width 0.6) (layer B.Cu) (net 5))
 (segment (start 46.99 33.02) (end 43.18 36.83) (width 0.6) (layer B.Cu) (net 5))
 (segment (start 46.355 45.085) (end 68.58 45.085) (width 0.6) (layer B.Cu) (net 5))
 (segment (start 43.18 41.91) (end 46.355 45.085) (width 0.6) (layer B.Cu) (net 5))
 (segment (start 43.18 36.83) (end 43.18 41.91) (width 0.6) (layer B.Cu) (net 5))
 (segment (start 46.99 33.02) (end 40.64 33.02) (width 0.6) (layer B.Cu) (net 5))
 (segment (start 51.435 91.44) (end 58.42 91.44) (width 0.6) (layer B.Cu) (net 5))
 (segment (start 73.66 40.005) (end 77.47 40.005) (width 0.6) (layer B.Cu) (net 6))
 (segment (start 69.85 40.005) (end 73.66 40.005) (width 0.6) (layer B.Cu) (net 6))
 (segment (start 46.99 130.81) (end 45.085 130.81) (width 0.6) (layer B.Cu) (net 14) (status 400000))
 (segment (start 54.61 137.16) (end 57.785 133.985) (width 0.6) (layer B.Cu) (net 14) (status 800000))
 (segment (start 46.355 137.16) (end 54.61 137.16) (width 0.6) (layer B.Cu) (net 14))
 (segment (start 44.45 135.255) (end 46.355 137.16) (width 0.6) (layer B.Cu) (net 14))
 (segment (start 44.45 131.445) (end 44.45 135.255) (width 0.6) (layer B.Cu) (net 14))
 (segment (start 45.085 130.81) (end 44.45 131.445) (width 0.6) (layer B.Cu) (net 14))
 (segment (start 46.99 48.26) (end 45.72 48.26) (width 0.6) (layer B.Cu) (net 8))
 (segment (start 45.72 48.26) (end 40.64 43.18) (width 0.6) (layer B.Cu) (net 8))
 (segment (start 85.725 38.1) (end 85.725 41.91) (width 0.6) (layer B.Cu) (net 9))
 (segment (start 85.725 41.91) (end 86.995 43.18) (width 0.6) (layer B.Cu) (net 9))
 (segment (start 85.09 43.18) (end 86.995 43.18) (width 0.6) (layer B.Cu) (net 9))
 (segment (start 81.788 43.18) (end 49.53 43.18) (width 0.6) (layer B.Cu) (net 9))
 (segment (start 49.53 43.18) (end 46.99 40.64) (width 0.6) (layer B.Cu) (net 9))
 (segment (start 81.788 43.18) (end 85.09 43.18) (width 0.6) (layer B.Cu) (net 9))
 (segment (start 85.09 43.18) (end 85.852 43.18) (width 0.6) (layer B.Cu) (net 9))
 (segment (start 58.42 36.83) (end 54.61 36.83) (width 0.6) (layer B.Cu) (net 9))
 (segment (start 54.61 36.83) (end 50.8 40.64) (width 0.6) (layer B.Cu) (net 9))
 (segment (start 46.99 40.64) (end 50.8 40.64) (width 0.6) (layer B.Cu) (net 9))
 (segment (start 51.435 83.82) (end 58.42 83.82) (width 0.6) (layer B.Cu) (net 12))
 (segment (start 81.915 24.765) (end 80.645 24.765) (width 0.6) (layer B.Cu) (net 11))
 (segment (start 90.17 33.655) (end 86.36 29.845) (width 0.6) (layer B.Cu) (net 11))
 (segment (start 86.36 29.845) (end 86.36 29.21) (width 0.6) (layer B.Cu) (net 11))
 (segment (start 86.36 29.21) (end 81.915 24.765) (width 0.6) (layer B.Cu) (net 11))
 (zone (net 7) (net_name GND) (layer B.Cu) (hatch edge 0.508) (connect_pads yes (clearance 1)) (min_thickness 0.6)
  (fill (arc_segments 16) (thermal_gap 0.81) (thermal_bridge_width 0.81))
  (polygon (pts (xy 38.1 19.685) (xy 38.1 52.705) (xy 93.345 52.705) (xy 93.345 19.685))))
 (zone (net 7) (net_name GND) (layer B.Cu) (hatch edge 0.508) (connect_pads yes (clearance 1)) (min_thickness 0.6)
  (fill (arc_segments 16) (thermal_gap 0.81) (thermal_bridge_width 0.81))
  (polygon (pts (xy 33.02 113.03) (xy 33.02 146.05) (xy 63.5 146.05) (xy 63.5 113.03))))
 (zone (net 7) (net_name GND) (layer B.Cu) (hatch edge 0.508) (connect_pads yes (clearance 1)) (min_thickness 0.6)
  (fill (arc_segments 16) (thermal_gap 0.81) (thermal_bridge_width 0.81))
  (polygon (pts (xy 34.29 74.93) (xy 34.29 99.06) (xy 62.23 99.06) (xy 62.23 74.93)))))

